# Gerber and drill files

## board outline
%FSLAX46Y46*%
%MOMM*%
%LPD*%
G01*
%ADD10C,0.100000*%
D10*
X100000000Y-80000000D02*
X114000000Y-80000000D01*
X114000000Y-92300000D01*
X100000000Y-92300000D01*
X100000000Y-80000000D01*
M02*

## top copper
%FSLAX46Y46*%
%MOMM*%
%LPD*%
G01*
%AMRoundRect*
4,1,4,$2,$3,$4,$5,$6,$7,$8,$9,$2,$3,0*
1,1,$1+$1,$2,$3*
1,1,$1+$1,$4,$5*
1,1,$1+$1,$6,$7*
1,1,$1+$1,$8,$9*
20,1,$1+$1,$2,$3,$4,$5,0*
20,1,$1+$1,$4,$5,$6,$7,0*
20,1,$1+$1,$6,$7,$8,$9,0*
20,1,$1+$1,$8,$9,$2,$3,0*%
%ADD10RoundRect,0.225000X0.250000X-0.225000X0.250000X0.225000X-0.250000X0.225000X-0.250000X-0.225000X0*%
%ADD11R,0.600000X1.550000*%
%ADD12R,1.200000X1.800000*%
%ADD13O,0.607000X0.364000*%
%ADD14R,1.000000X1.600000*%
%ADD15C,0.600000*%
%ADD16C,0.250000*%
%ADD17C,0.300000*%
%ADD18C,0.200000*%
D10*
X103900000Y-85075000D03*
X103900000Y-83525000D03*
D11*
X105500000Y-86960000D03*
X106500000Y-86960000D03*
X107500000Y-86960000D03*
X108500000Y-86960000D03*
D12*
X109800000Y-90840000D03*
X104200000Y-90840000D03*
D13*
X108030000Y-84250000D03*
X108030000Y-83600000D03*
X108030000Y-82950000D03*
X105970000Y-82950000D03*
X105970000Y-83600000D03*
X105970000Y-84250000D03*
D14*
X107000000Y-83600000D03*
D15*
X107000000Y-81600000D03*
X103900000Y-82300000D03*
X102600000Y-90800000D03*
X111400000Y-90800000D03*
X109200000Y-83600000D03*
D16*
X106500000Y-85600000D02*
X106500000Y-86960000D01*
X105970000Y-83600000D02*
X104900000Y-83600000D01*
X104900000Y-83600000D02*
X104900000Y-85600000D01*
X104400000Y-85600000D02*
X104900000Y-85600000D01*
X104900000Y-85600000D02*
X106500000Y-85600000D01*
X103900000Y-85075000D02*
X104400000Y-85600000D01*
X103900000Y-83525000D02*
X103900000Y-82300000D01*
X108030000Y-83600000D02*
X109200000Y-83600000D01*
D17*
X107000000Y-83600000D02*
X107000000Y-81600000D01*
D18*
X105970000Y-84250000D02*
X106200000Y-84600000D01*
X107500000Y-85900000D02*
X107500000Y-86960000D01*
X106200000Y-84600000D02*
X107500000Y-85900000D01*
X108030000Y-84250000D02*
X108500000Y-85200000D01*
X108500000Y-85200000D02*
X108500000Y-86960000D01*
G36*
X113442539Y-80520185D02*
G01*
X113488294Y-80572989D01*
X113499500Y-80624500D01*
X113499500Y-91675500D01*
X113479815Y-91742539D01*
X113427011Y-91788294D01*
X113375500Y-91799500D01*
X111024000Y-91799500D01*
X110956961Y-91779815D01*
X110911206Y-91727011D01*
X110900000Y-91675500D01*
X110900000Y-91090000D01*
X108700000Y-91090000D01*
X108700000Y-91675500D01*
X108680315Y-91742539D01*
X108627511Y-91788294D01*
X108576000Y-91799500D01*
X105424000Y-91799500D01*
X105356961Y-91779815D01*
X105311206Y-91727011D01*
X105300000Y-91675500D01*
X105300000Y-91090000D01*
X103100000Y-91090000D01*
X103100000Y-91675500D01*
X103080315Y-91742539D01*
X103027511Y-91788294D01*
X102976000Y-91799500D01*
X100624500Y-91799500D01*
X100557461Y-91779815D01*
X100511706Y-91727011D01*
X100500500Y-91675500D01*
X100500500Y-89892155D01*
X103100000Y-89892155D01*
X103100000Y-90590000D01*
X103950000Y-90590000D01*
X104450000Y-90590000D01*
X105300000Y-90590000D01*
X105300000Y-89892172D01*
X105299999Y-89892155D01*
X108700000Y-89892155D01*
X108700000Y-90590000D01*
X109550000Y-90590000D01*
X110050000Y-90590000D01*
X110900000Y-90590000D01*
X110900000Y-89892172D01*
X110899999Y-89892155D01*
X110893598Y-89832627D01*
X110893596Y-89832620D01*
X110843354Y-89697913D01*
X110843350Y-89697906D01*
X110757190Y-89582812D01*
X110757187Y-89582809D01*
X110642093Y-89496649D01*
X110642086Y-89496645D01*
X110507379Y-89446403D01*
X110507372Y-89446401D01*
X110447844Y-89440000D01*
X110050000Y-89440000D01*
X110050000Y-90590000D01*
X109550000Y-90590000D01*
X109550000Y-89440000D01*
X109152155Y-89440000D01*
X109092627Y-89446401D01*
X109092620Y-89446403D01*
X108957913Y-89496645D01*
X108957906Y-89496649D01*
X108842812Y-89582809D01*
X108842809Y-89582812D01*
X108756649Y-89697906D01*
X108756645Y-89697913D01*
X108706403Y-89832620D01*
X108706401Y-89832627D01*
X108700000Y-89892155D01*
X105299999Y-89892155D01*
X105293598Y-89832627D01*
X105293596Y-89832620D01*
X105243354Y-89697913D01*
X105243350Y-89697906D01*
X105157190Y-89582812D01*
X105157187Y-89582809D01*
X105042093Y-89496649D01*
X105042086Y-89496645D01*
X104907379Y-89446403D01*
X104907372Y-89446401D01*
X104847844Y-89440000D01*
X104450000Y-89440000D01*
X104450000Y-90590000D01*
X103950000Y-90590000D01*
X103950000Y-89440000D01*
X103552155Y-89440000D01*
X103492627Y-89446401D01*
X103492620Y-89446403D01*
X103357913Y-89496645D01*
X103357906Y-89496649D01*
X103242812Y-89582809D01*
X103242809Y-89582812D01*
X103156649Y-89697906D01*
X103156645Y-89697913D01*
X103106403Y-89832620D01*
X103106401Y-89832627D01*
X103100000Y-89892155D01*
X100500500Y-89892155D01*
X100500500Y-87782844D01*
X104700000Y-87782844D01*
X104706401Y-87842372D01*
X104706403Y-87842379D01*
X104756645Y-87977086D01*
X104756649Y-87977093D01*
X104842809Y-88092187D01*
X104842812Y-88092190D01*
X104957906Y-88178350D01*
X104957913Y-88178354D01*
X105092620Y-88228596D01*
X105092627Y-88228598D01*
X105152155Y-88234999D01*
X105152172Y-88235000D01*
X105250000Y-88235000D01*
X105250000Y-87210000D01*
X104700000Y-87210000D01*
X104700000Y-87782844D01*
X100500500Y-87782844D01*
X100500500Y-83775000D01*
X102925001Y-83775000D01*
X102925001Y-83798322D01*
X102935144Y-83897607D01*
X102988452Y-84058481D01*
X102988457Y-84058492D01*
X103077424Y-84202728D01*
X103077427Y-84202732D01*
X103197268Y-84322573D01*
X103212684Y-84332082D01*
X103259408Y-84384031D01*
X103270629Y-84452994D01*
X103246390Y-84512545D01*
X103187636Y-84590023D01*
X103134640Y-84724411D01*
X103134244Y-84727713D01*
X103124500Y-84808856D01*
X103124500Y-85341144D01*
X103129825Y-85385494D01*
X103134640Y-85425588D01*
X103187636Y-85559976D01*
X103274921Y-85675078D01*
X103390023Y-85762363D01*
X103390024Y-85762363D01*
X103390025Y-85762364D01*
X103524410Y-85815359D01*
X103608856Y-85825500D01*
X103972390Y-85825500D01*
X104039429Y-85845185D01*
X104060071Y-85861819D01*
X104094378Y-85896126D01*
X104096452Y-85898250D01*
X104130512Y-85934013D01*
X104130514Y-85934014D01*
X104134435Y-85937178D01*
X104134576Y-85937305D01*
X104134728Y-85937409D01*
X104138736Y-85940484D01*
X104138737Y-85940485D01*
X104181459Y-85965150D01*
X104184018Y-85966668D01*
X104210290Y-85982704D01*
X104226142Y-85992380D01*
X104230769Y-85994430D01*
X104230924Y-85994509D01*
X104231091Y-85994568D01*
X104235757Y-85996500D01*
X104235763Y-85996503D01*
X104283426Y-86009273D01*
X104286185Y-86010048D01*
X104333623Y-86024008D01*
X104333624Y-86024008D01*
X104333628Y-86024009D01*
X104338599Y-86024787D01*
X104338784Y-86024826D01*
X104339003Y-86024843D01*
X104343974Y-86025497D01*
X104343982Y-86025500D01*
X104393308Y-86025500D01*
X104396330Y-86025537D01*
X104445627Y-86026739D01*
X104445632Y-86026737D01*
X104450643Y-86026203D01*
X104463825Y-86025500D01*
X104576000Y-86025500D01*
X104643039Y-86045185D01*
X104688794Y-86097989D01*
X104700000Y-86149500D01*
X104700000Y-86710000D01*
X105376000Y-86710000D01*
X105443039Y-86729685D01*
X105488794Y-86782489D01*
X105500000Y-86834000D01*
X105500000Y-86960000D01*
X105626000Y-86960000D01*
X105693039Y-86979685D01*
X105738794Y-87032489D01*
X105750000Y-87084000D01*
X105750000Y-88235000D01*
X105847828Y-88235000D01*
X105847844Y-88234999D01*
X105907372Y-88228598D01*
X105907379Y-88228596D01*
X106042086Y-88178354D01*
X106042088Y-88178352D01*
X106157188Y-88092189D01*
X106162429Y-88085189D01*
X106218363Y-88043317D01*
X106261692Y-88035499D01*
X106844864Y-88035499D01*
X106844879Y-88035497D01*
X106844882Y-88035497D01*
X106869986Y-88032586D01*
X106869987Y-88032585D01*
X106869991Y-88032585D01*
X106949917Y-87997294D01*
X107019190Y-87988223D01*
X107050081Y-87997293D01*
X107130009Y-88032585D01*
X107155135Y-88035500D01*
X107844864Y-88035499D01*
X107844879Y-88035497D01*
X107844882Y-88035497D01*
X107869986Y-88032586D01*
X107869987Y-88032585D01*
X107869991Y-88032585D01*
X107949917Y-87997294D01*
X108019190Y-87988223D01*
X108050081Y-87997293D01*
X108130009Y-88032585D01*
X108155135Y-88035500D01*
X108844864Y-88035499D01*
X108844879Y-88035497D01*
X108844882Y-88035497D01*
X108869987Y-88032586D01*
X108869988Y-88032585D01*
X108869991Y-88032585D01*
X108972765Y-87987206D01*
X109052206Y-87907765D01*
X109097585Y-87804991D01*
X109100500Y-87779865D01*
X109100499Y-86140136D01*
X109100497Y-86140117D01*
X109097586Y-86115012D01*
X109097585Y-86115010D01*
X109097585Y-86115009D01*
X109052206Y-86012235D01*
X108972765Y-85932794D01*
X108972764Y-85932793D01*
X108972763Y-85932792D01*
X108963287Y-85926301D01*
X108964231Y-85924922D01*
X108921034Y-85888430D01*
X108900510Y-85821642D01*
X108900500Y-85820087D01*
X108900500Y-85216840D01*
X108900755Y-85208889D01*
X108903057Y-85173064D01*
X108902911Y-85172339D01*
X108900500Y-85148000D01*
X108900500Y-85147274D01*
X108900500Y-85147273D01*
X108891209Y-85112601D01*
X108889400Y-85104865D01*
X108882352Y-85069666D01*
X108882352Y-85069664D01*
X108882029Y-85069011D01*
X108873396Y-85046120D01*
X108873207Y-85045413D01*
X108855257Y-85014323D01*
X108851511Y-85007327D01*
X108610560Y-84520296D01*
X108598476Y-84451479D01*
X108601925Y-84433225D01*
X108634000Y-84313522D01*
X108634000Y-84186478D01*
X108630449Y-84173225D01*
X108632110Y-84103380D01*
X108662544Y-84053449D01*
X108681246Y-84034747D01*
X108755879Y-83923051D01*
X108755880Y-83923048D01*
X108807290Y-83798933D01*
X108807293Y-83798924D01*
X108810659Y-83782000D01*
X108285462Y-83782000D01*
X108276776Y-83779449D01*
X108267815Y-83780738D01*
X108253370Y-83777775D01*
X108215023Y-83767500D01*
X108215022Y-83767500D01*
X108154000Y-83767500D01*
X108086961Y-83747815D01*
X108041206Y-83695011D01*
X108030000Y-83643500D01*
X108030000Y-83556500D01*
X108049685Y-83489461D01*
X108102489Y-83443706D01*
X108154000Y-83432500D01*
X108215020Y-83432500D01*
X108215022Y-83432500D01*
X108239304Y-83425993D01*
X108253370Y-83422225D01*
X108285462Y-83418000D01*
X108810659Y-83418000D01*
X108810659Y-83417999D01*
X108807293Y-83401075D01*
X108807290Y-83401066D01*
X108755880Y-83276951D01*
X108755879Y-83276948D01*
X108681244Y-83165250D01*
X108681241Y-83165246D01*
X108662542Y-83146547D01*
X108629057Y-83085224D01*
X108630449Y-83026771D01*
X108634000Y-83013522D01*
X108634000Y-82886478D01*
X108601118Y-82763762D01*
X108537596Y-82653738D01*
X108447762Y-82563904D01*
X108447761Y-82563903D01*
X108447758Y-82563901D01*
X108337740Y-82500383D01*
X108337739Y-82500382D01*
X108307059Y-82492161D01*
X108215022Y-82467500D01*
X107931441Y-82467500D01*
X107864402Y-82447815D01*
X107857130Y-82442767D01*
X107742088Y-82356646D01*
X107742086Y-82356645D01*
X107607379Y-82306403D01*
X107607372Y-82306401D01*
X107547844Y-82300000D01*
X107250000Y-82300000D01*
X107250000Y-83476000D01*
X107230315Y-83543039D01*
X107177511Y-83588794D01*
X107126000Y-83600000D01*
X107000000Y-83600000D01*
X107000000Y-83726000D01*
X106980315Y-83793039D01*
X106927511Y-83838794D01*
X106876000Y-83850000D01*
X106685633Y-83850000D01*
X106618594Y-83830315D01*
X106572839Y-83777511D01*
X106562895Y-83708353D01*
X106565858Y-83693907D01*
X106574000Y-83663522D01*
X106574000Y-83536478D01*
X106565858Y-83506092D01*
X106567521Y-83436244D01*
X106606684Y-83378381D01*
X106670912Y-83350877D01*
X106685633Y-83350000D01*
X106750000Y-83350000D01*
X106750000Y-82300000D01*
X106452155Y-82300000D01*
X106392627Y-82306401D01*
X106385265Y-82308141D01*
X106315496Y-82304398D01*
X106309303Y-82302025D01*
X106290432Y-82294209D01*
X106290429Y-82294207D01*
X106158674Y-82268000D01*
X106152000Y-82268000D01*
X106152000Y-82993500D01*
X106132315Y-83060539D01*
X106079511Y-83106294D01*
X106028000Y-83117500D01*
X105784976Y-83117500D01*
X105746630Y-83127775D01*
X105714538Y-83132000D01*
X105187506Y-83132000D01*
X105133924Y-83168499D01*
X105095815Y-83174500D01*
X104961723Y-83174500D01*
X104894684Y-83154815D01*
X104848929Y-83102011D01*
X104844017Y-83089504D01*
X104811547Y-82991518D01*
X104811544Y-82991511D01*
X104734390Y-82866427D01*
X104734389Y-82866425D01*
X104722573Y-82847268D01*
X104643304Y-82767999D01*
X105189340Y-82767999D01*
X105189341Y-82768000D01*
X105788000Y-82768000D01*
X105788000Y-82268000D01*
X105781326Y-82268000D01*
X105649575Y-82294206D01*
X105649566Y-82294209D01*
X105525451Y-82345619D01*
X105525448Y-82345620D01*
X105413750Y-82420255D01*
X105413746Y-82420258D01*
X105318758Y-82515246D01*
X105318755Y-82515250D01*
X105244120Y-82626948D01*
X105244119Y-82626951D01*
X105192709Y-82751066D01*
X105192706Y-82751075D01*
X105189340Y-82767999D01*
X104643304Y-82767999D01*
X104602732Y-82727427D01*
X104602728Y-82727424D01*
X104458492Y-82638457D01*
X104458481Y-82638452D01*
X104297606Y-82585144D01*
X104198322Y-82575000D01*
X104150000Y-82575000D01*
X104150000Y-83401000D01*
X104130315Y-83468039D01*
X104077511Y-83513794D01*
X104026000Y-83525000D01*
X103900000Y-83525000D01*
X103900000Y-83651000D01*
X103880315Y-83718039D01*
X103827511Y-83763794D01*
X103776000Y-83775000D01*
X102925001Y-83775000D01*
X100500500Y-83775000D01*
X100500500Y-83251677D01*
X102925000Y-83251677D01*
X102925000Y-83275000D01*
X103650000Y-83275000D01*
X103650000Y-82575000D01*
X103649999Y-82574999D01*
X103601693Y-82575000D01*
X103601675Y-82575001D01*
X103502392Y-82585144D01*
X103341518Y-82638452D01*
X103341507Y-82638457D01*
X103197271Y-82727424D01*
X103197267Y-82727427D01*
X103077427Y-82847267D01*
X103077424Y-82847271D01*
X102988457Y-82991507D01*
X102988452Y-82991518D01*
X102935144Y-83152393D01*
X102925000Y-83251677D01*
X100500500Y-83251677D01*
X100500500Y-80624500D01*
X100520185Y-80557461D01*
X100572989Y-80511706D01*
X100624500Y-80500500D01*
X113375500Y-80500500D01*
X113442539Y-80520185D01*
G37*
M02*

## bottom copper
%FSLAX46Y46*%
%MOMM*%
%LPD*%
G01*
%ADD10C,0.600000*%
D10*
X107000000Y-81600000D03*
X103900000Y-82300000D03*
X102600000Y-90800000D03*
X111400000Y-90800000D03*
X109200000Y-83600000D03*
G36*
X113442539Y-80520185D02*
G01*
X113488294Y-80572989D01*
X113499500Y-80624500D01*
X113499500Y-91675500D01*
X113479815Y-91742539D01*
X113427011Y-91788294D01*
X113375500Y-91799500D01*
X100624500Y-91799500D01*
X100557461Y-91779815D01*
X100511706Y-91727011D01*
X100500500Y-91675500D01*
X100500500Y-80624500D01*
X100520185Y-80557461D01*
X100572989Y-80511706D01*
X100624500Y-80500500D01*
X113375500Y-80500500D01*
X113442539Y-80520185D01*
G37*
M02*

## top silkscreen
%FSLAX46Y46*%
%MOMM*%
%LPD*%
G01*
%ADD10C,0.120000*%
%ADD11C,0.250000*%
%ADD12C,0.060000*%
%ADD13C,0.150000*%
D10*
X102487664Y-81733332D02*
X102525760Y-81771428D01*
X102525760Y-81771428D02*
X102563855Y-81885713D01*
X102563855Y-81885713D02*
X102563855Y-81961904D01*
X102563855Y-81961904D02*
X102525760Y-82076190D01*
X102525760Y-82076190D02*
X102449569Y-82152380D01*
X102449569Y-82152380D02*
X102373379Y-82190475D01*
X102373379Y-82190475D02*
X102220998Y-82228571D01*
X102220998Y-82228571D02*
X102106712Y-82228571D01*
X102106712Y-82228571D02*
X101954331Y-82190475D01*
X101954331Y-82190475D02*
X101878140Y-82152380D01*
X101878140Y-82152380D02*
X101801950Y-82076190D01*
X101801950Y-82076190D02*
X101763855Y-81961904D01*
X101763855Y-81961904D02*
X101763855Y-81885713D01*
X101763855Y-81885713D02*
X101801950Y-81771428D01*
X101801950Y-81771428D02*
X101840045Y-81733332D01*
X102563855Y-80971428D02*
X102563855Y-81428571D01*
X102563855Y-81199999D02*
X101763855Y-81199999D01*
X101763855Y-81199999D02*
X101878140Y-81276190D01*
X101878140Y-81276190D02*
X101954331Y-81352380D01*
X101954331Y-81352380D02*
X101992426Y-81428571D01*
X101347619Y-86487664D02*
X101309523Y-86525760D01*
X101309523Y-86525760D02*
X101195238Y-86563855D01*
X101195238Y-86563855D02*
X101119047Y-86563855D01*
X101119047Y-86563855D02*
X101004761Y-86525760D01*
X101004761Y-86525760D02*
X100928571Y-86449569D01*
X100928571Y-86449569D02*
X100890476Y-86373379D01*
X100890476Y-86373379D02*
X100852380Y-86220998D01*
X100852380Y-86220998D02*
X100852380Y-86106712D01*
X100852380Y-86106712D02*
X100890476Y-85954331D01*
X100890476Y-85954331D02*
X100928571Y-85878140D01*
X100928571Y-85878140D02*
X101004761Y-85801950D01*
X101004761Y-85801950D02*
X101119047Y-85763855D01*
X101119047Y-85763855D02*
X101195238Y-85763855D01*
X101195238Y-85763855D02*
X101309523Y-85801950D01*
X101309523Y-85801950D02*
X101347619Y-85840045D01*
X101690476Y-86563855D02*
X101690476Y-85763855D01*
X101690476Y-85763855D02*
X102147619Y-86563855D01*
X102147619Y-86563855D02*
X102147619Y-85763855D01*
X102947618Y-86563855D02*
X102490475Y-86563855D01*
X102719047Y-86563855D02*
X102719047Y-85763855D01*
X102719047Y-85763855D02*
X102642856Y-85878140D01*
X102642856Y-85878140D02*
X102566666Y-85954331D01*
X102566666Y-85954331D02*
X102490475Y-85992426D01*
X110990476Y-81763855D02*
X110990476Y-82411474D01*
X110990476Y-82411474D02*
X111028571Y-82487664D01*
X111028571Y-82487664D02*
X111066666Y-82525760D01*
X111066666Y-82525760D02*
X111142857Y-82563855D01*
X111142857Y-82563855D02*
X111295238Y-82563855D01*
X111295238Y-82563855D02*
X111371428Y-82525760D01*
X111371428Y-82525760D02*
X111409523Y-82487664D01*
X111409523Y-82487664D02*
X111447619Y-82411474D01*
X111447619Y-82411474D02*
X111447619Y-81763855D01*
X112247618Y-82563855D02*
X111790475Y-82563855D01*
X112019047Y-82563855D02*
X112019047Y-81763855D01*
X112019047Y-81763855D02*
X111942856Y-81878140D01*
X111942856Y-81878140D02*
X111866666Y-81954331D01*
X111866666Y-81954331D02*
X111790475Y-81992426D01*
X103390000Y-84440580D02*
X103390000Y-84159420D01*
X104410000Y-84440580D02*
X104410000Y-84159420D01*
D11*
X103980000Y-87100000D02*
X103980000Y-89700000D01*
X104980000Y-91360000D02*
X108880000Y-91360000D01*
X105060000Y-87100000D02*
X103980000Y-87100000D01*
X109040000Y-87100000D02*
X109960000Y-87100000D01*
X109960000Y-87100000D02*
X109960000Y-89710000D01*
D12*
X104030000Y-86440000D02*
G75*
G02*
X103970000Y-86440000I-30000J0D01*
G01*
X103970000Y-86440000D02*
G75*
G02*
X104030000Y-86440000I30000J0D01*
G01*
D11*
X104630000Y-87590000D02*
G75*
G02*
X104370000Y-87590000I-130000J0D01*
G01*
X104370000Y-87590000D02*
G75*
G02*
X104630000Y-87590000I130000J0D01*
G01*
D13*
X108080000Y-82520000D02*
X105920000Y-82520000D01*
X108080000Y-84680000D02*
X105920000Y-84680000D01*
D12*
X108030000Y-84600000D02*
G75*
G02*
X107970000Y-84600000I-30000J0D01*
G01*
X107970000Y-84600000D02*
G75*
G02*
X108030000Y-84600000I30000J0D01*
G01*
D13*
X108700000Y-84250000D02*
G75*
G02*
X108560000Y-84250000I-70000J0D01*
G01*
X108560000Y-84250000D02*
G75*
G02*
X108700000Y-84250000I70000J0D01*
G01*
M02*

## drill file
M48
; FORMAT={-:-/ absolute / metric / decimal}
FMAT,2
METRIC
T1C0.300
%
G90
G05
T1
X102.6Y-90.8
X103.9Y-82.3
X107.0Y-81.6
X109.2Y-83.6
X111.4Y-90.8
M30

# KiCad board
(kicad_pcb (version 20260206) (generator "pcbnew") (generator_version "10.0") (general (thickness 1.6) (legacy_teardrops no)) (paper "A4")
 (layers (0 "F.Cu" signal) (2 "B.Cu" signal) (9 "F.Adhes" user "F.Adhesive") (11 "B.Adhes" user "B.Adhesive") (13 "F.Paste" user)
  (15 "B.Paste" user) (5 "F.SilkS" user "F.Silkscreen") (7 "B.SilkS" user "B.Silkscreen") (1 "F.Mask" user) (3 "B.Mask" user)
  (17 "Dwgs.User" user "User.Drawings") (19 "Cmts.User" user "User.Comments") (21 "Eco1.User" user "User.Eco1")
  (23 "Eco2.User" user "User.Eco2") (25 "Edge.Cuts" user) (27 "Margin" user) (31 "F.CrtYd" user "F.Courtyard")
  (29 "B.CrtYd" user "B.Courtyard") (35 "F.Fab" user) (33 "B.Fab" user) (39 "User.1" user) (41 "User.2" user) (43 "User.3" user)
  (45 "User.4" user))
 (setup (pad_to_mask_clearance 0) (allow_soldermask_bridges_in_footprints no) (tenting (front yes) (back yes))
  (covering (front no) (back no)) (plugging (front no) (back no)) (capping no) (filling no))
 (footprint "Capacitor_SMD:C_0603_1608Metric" (layer "F.Cu") (at 103.9 84.3 90)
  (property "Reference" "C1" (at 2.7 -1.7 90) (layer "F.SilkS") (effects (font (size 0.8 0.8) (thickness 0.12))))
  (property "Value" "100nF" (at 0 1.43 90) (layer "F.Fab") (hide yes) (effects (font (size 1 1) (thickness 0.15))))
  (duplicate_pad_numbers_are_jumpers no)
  (fp_line (start -0.14058 -0.51) (end 0.14058 -0.51) (stroke (width 0.12) (type solid)) (layer "F.SilkS"))
  (fp_line (start -0.14058 0.51) (end 0.14058 0.51) (stroke (width 0.12) (type solid)) (layer "F.SilkS"))
  (pad "1" smd roundrect (at -0.775 0 90) (size 0.9 0.95) (layers "F.Cu" "F.Mask" "F.Paste") (roundrect_rratio 0.25) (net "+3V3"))
  (pad "2" smd roundrect (at 0.775 0 90) (size 0.9 0.95) (layers "F.Cu" "F.Mask" "F.Paste") (roundrect_rratio 0.25) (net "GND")))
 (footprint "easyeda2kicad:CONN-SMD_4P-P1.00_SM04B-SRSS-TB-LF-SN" (layer "F.Cu") (at 107 88.9)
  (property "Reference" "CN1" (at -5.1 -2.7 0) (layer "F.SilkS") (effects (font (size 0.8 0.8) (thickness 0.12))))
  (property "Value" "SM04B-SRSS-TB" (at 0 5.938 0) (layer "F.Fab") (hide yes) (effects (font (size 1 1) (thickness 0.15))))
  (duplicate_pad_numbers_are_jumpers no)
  (fp_line (start -3.02 -1.8) (end -3.02 0.8) (stroke (width 0.25) (type solid)) (layer "F.SilkS"))
  (fp_line (start -2.02 2.46) (end 1.88 2.46) (stroke (width 0.25) (type solid)) (layer "F.SilkS"))
  (fp_line (start -1.94 -1.8) (end -3.02 -1.8) (stroke (width 0.25) (type solid)) (layer "F.SilkS"))
  (fp_line (start 2.04 -1.8) (end 2.96 -1.8) (stroke (width 0.25) (type solid)) (layer "F.SilkS"))
  (fp_line (start 2.96 -1.8) (end 2.96 0.81) (stroke (width 0.25) (type solid)) (layer "F.SilkS"))
  (fp_circle (center -3 -2.46) (end -2.97 -2.46) (stroke (width 0.06) (type solid)) (fill no) (layer "F.SilkS"))
  (fp_circle (center -2.5 -1.31) (end -2.37 -1.31) (stroke (width 0.25) (type solid)) (fill no) (layer "F.SilkS"))
  (pad "1" smd rect (at -1.5 -1.94) (size 0.6 1.55) (layers "F.Cu" "F.Mask" "F.Paste") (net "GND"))
  (pad "2" smd rect (at -0.5 -1.94) (size 0.6 1.55) (layers "F.Cu" "F.Mask" "F.Paste") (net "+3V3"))
  (pad "3" smd rect (at 0.5 -1.94) (size 0.6 1.55) (layers "F.Cu" "F.Mask" "F.Paste") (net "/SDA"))
  (pad "4" smd rect (at 1.5 -1.94) (size 0.6 1.55) (layers "F.Cu" "F.Mask" "F.Paste") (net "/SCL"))
  (pad "5" smd rect (at 2.8 1.94) (size 1.2 1.8) (layers "F.Cu" "F.Mask" "F.Paste") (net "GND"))
  (pad "6" smd rect (at -2.8 1.94) (size 1.2 1.8) (layers "F.Cu" "F.Mask" "F.Paste") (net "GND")))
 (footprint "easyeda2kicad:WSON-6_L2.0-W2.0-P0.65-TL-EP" (layer "F.Cu") (at 107 83.6 180)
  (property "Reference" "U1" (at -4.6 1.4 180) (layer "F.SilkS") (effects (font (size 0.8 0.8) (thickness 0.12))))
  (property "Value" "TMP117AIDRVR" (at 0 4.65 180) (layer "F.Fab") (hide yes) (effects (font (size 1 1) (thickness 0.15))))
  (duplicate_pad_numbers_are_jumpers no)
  (fp_line (start -1.08 1.08) (end 1.08 1.08) (stroke (width 0.15) (type solid)) (layer "F.SilkS"))
  (fp_line (start -1.08 -1.08) (end 1.08 -1.08) (stroke (width 0.15) (type solid)) (layer "F.SilkS"))
  (fp_circle (center -1 -1) (end -0.97 -1) (stroke (width 0.06) (type solid)) (fill no) (layer "F.SilkS"))
  (fp_circle (center -1.63 -0.65) (end -1.56 -0.65) (stroke (width 0.15) (type solid)) (fill no) (layer "F.SilkS"))
  (pad "1" smd oval (at -1.03 -0.65 90) (size 0.364 0.607) (layers "F.Cu" "F.Mask" "F.Paste") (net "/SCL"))
  (pad "2" smd oval (at -1.03 0 90) (size 0.364 0.607) (layers "F.Cu" "F.Mask" "F.Paste") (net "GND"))
  (pad "3" smd oval (at -1.03 0.65 90) (size 0.364 0.607) (layers "F.Cu" "F.Mask" "F.Paste") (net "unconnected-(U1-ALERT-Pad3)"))
  (pad "4" smd oval (at 1.03 0.65 90) (size 0.364 0.607) (layers "F.Cu" "F.Mask" "F.Paste") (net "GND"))
  (pad "5" smd oval (at 1.03 0 90) (size 0.364 0.607) (layers "F.Cu" "F.Mask" "F.Paste") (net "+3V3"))
  (pad "6" smd oval (at 1.03 -0.65 90) (size 0.364 0.607) (layers "F.Cu" "F.Mask" "F.Paste") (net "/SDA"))
  (pad "7" smd rect (at 0 0 180) (size 1 1.6) (layers "F.Cu" "F.Mask" "F.Paste") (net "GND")))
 (gr_rect (start 100 80) (end 114 92.3) (stroke (width 0.1) (type default)) (fill no) (layer "Edge.Cuts"))
 (segment (start 106.5 85.6) (end 106.5 86.96) (width 0.25) (layer "F.Cu") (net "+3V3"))
 (segment (start 105.97 83.6) (end 104.9 83.6) (width 0.25) (layer "F.Cu") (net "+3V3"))
 (segment (start 104.9 83.6) (end 104.9 85.6) (width 0.25) (layer "F.Cu") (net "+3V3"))
 (segment (start 104.4 85.6) (end 104.9 85.6) (width 0.25) (layer "F.Cu") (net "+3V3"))
 (segment (start 104.9 85.6) (end 106.5 85.6) (width 0.25) (layer "F.Cu") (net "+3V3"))
 (segment (start 103.9 85.075) (end 104.4 85.6) (width 0.25) (layer "F.Cu") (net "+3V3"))
 (segment (start 103.9 83.525) (end 103.9 82.3) (width 0.25) (layer "F.Cu") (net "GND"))
 (segment (start 108.03 83.6) (end 109.2 83.6) (width 0.25) (layer "F.Cu") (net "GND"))
 (segment (start 107 83.6) (end 107 81.6) (width 0.3) (layer "F.Cu") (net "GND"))
 (via (at 107 81.6) (size 0.6) (drill 0.3) (layers "F.Cu" "B.Cu") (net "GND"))
 (via (at 103.9 82.3) (size 0.6) (drill 0.3) (layers "F.Cu" "B.Cu") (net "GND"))
 (via (at 102.6 90.8) (size 0.6) (drill 0.3) (layers "F.Cu" "B.Cu") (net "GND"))
 (via (at 111.4 90.8) (size 0.6) (drill 0.3) (layers "F.Cu" "B.Cu") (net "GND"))
 (via (at 109.2 83.6) (size 0.6) (drill 0.3) (layers "F.Cu" "B.Cu") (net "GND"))
 (segment (start 105.97 84.25) (end 106.2 84.6) (width 0.2) (layer "F.Cu") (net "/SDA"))
 (segment (start 107.5 85.9) (end 107.5 86.96) (width 0.2) (layer "F.Cu") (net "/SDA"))
 (segment (start 106.2 84.6) (end 107.5 85.9) (width 0.2) (layer "F.Cu") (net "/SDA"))
 (segment (start 108.03 84.25) (end 108.5 85.2) (width 0.2) (layer "F.Cu") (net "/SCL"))
 (segment (start 108.5 85.2) (end 108.5 86.96) (width 0.2) (layer "F.Cu") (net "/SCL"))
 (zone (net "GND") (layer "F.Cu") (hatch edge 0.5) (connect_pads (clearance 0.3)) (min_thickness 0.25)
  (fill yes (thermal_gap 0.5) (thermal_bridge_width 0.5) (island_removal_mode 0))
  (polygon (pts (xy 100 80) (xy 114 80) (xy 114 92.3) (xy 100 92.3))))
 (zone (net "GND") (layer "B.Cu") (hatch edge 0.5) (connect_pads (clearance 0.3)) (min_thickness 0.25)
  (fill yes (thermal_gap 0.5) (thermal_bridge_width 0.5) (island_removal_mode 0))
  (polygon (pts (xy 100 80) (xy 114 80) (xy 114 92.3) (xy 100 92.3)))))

